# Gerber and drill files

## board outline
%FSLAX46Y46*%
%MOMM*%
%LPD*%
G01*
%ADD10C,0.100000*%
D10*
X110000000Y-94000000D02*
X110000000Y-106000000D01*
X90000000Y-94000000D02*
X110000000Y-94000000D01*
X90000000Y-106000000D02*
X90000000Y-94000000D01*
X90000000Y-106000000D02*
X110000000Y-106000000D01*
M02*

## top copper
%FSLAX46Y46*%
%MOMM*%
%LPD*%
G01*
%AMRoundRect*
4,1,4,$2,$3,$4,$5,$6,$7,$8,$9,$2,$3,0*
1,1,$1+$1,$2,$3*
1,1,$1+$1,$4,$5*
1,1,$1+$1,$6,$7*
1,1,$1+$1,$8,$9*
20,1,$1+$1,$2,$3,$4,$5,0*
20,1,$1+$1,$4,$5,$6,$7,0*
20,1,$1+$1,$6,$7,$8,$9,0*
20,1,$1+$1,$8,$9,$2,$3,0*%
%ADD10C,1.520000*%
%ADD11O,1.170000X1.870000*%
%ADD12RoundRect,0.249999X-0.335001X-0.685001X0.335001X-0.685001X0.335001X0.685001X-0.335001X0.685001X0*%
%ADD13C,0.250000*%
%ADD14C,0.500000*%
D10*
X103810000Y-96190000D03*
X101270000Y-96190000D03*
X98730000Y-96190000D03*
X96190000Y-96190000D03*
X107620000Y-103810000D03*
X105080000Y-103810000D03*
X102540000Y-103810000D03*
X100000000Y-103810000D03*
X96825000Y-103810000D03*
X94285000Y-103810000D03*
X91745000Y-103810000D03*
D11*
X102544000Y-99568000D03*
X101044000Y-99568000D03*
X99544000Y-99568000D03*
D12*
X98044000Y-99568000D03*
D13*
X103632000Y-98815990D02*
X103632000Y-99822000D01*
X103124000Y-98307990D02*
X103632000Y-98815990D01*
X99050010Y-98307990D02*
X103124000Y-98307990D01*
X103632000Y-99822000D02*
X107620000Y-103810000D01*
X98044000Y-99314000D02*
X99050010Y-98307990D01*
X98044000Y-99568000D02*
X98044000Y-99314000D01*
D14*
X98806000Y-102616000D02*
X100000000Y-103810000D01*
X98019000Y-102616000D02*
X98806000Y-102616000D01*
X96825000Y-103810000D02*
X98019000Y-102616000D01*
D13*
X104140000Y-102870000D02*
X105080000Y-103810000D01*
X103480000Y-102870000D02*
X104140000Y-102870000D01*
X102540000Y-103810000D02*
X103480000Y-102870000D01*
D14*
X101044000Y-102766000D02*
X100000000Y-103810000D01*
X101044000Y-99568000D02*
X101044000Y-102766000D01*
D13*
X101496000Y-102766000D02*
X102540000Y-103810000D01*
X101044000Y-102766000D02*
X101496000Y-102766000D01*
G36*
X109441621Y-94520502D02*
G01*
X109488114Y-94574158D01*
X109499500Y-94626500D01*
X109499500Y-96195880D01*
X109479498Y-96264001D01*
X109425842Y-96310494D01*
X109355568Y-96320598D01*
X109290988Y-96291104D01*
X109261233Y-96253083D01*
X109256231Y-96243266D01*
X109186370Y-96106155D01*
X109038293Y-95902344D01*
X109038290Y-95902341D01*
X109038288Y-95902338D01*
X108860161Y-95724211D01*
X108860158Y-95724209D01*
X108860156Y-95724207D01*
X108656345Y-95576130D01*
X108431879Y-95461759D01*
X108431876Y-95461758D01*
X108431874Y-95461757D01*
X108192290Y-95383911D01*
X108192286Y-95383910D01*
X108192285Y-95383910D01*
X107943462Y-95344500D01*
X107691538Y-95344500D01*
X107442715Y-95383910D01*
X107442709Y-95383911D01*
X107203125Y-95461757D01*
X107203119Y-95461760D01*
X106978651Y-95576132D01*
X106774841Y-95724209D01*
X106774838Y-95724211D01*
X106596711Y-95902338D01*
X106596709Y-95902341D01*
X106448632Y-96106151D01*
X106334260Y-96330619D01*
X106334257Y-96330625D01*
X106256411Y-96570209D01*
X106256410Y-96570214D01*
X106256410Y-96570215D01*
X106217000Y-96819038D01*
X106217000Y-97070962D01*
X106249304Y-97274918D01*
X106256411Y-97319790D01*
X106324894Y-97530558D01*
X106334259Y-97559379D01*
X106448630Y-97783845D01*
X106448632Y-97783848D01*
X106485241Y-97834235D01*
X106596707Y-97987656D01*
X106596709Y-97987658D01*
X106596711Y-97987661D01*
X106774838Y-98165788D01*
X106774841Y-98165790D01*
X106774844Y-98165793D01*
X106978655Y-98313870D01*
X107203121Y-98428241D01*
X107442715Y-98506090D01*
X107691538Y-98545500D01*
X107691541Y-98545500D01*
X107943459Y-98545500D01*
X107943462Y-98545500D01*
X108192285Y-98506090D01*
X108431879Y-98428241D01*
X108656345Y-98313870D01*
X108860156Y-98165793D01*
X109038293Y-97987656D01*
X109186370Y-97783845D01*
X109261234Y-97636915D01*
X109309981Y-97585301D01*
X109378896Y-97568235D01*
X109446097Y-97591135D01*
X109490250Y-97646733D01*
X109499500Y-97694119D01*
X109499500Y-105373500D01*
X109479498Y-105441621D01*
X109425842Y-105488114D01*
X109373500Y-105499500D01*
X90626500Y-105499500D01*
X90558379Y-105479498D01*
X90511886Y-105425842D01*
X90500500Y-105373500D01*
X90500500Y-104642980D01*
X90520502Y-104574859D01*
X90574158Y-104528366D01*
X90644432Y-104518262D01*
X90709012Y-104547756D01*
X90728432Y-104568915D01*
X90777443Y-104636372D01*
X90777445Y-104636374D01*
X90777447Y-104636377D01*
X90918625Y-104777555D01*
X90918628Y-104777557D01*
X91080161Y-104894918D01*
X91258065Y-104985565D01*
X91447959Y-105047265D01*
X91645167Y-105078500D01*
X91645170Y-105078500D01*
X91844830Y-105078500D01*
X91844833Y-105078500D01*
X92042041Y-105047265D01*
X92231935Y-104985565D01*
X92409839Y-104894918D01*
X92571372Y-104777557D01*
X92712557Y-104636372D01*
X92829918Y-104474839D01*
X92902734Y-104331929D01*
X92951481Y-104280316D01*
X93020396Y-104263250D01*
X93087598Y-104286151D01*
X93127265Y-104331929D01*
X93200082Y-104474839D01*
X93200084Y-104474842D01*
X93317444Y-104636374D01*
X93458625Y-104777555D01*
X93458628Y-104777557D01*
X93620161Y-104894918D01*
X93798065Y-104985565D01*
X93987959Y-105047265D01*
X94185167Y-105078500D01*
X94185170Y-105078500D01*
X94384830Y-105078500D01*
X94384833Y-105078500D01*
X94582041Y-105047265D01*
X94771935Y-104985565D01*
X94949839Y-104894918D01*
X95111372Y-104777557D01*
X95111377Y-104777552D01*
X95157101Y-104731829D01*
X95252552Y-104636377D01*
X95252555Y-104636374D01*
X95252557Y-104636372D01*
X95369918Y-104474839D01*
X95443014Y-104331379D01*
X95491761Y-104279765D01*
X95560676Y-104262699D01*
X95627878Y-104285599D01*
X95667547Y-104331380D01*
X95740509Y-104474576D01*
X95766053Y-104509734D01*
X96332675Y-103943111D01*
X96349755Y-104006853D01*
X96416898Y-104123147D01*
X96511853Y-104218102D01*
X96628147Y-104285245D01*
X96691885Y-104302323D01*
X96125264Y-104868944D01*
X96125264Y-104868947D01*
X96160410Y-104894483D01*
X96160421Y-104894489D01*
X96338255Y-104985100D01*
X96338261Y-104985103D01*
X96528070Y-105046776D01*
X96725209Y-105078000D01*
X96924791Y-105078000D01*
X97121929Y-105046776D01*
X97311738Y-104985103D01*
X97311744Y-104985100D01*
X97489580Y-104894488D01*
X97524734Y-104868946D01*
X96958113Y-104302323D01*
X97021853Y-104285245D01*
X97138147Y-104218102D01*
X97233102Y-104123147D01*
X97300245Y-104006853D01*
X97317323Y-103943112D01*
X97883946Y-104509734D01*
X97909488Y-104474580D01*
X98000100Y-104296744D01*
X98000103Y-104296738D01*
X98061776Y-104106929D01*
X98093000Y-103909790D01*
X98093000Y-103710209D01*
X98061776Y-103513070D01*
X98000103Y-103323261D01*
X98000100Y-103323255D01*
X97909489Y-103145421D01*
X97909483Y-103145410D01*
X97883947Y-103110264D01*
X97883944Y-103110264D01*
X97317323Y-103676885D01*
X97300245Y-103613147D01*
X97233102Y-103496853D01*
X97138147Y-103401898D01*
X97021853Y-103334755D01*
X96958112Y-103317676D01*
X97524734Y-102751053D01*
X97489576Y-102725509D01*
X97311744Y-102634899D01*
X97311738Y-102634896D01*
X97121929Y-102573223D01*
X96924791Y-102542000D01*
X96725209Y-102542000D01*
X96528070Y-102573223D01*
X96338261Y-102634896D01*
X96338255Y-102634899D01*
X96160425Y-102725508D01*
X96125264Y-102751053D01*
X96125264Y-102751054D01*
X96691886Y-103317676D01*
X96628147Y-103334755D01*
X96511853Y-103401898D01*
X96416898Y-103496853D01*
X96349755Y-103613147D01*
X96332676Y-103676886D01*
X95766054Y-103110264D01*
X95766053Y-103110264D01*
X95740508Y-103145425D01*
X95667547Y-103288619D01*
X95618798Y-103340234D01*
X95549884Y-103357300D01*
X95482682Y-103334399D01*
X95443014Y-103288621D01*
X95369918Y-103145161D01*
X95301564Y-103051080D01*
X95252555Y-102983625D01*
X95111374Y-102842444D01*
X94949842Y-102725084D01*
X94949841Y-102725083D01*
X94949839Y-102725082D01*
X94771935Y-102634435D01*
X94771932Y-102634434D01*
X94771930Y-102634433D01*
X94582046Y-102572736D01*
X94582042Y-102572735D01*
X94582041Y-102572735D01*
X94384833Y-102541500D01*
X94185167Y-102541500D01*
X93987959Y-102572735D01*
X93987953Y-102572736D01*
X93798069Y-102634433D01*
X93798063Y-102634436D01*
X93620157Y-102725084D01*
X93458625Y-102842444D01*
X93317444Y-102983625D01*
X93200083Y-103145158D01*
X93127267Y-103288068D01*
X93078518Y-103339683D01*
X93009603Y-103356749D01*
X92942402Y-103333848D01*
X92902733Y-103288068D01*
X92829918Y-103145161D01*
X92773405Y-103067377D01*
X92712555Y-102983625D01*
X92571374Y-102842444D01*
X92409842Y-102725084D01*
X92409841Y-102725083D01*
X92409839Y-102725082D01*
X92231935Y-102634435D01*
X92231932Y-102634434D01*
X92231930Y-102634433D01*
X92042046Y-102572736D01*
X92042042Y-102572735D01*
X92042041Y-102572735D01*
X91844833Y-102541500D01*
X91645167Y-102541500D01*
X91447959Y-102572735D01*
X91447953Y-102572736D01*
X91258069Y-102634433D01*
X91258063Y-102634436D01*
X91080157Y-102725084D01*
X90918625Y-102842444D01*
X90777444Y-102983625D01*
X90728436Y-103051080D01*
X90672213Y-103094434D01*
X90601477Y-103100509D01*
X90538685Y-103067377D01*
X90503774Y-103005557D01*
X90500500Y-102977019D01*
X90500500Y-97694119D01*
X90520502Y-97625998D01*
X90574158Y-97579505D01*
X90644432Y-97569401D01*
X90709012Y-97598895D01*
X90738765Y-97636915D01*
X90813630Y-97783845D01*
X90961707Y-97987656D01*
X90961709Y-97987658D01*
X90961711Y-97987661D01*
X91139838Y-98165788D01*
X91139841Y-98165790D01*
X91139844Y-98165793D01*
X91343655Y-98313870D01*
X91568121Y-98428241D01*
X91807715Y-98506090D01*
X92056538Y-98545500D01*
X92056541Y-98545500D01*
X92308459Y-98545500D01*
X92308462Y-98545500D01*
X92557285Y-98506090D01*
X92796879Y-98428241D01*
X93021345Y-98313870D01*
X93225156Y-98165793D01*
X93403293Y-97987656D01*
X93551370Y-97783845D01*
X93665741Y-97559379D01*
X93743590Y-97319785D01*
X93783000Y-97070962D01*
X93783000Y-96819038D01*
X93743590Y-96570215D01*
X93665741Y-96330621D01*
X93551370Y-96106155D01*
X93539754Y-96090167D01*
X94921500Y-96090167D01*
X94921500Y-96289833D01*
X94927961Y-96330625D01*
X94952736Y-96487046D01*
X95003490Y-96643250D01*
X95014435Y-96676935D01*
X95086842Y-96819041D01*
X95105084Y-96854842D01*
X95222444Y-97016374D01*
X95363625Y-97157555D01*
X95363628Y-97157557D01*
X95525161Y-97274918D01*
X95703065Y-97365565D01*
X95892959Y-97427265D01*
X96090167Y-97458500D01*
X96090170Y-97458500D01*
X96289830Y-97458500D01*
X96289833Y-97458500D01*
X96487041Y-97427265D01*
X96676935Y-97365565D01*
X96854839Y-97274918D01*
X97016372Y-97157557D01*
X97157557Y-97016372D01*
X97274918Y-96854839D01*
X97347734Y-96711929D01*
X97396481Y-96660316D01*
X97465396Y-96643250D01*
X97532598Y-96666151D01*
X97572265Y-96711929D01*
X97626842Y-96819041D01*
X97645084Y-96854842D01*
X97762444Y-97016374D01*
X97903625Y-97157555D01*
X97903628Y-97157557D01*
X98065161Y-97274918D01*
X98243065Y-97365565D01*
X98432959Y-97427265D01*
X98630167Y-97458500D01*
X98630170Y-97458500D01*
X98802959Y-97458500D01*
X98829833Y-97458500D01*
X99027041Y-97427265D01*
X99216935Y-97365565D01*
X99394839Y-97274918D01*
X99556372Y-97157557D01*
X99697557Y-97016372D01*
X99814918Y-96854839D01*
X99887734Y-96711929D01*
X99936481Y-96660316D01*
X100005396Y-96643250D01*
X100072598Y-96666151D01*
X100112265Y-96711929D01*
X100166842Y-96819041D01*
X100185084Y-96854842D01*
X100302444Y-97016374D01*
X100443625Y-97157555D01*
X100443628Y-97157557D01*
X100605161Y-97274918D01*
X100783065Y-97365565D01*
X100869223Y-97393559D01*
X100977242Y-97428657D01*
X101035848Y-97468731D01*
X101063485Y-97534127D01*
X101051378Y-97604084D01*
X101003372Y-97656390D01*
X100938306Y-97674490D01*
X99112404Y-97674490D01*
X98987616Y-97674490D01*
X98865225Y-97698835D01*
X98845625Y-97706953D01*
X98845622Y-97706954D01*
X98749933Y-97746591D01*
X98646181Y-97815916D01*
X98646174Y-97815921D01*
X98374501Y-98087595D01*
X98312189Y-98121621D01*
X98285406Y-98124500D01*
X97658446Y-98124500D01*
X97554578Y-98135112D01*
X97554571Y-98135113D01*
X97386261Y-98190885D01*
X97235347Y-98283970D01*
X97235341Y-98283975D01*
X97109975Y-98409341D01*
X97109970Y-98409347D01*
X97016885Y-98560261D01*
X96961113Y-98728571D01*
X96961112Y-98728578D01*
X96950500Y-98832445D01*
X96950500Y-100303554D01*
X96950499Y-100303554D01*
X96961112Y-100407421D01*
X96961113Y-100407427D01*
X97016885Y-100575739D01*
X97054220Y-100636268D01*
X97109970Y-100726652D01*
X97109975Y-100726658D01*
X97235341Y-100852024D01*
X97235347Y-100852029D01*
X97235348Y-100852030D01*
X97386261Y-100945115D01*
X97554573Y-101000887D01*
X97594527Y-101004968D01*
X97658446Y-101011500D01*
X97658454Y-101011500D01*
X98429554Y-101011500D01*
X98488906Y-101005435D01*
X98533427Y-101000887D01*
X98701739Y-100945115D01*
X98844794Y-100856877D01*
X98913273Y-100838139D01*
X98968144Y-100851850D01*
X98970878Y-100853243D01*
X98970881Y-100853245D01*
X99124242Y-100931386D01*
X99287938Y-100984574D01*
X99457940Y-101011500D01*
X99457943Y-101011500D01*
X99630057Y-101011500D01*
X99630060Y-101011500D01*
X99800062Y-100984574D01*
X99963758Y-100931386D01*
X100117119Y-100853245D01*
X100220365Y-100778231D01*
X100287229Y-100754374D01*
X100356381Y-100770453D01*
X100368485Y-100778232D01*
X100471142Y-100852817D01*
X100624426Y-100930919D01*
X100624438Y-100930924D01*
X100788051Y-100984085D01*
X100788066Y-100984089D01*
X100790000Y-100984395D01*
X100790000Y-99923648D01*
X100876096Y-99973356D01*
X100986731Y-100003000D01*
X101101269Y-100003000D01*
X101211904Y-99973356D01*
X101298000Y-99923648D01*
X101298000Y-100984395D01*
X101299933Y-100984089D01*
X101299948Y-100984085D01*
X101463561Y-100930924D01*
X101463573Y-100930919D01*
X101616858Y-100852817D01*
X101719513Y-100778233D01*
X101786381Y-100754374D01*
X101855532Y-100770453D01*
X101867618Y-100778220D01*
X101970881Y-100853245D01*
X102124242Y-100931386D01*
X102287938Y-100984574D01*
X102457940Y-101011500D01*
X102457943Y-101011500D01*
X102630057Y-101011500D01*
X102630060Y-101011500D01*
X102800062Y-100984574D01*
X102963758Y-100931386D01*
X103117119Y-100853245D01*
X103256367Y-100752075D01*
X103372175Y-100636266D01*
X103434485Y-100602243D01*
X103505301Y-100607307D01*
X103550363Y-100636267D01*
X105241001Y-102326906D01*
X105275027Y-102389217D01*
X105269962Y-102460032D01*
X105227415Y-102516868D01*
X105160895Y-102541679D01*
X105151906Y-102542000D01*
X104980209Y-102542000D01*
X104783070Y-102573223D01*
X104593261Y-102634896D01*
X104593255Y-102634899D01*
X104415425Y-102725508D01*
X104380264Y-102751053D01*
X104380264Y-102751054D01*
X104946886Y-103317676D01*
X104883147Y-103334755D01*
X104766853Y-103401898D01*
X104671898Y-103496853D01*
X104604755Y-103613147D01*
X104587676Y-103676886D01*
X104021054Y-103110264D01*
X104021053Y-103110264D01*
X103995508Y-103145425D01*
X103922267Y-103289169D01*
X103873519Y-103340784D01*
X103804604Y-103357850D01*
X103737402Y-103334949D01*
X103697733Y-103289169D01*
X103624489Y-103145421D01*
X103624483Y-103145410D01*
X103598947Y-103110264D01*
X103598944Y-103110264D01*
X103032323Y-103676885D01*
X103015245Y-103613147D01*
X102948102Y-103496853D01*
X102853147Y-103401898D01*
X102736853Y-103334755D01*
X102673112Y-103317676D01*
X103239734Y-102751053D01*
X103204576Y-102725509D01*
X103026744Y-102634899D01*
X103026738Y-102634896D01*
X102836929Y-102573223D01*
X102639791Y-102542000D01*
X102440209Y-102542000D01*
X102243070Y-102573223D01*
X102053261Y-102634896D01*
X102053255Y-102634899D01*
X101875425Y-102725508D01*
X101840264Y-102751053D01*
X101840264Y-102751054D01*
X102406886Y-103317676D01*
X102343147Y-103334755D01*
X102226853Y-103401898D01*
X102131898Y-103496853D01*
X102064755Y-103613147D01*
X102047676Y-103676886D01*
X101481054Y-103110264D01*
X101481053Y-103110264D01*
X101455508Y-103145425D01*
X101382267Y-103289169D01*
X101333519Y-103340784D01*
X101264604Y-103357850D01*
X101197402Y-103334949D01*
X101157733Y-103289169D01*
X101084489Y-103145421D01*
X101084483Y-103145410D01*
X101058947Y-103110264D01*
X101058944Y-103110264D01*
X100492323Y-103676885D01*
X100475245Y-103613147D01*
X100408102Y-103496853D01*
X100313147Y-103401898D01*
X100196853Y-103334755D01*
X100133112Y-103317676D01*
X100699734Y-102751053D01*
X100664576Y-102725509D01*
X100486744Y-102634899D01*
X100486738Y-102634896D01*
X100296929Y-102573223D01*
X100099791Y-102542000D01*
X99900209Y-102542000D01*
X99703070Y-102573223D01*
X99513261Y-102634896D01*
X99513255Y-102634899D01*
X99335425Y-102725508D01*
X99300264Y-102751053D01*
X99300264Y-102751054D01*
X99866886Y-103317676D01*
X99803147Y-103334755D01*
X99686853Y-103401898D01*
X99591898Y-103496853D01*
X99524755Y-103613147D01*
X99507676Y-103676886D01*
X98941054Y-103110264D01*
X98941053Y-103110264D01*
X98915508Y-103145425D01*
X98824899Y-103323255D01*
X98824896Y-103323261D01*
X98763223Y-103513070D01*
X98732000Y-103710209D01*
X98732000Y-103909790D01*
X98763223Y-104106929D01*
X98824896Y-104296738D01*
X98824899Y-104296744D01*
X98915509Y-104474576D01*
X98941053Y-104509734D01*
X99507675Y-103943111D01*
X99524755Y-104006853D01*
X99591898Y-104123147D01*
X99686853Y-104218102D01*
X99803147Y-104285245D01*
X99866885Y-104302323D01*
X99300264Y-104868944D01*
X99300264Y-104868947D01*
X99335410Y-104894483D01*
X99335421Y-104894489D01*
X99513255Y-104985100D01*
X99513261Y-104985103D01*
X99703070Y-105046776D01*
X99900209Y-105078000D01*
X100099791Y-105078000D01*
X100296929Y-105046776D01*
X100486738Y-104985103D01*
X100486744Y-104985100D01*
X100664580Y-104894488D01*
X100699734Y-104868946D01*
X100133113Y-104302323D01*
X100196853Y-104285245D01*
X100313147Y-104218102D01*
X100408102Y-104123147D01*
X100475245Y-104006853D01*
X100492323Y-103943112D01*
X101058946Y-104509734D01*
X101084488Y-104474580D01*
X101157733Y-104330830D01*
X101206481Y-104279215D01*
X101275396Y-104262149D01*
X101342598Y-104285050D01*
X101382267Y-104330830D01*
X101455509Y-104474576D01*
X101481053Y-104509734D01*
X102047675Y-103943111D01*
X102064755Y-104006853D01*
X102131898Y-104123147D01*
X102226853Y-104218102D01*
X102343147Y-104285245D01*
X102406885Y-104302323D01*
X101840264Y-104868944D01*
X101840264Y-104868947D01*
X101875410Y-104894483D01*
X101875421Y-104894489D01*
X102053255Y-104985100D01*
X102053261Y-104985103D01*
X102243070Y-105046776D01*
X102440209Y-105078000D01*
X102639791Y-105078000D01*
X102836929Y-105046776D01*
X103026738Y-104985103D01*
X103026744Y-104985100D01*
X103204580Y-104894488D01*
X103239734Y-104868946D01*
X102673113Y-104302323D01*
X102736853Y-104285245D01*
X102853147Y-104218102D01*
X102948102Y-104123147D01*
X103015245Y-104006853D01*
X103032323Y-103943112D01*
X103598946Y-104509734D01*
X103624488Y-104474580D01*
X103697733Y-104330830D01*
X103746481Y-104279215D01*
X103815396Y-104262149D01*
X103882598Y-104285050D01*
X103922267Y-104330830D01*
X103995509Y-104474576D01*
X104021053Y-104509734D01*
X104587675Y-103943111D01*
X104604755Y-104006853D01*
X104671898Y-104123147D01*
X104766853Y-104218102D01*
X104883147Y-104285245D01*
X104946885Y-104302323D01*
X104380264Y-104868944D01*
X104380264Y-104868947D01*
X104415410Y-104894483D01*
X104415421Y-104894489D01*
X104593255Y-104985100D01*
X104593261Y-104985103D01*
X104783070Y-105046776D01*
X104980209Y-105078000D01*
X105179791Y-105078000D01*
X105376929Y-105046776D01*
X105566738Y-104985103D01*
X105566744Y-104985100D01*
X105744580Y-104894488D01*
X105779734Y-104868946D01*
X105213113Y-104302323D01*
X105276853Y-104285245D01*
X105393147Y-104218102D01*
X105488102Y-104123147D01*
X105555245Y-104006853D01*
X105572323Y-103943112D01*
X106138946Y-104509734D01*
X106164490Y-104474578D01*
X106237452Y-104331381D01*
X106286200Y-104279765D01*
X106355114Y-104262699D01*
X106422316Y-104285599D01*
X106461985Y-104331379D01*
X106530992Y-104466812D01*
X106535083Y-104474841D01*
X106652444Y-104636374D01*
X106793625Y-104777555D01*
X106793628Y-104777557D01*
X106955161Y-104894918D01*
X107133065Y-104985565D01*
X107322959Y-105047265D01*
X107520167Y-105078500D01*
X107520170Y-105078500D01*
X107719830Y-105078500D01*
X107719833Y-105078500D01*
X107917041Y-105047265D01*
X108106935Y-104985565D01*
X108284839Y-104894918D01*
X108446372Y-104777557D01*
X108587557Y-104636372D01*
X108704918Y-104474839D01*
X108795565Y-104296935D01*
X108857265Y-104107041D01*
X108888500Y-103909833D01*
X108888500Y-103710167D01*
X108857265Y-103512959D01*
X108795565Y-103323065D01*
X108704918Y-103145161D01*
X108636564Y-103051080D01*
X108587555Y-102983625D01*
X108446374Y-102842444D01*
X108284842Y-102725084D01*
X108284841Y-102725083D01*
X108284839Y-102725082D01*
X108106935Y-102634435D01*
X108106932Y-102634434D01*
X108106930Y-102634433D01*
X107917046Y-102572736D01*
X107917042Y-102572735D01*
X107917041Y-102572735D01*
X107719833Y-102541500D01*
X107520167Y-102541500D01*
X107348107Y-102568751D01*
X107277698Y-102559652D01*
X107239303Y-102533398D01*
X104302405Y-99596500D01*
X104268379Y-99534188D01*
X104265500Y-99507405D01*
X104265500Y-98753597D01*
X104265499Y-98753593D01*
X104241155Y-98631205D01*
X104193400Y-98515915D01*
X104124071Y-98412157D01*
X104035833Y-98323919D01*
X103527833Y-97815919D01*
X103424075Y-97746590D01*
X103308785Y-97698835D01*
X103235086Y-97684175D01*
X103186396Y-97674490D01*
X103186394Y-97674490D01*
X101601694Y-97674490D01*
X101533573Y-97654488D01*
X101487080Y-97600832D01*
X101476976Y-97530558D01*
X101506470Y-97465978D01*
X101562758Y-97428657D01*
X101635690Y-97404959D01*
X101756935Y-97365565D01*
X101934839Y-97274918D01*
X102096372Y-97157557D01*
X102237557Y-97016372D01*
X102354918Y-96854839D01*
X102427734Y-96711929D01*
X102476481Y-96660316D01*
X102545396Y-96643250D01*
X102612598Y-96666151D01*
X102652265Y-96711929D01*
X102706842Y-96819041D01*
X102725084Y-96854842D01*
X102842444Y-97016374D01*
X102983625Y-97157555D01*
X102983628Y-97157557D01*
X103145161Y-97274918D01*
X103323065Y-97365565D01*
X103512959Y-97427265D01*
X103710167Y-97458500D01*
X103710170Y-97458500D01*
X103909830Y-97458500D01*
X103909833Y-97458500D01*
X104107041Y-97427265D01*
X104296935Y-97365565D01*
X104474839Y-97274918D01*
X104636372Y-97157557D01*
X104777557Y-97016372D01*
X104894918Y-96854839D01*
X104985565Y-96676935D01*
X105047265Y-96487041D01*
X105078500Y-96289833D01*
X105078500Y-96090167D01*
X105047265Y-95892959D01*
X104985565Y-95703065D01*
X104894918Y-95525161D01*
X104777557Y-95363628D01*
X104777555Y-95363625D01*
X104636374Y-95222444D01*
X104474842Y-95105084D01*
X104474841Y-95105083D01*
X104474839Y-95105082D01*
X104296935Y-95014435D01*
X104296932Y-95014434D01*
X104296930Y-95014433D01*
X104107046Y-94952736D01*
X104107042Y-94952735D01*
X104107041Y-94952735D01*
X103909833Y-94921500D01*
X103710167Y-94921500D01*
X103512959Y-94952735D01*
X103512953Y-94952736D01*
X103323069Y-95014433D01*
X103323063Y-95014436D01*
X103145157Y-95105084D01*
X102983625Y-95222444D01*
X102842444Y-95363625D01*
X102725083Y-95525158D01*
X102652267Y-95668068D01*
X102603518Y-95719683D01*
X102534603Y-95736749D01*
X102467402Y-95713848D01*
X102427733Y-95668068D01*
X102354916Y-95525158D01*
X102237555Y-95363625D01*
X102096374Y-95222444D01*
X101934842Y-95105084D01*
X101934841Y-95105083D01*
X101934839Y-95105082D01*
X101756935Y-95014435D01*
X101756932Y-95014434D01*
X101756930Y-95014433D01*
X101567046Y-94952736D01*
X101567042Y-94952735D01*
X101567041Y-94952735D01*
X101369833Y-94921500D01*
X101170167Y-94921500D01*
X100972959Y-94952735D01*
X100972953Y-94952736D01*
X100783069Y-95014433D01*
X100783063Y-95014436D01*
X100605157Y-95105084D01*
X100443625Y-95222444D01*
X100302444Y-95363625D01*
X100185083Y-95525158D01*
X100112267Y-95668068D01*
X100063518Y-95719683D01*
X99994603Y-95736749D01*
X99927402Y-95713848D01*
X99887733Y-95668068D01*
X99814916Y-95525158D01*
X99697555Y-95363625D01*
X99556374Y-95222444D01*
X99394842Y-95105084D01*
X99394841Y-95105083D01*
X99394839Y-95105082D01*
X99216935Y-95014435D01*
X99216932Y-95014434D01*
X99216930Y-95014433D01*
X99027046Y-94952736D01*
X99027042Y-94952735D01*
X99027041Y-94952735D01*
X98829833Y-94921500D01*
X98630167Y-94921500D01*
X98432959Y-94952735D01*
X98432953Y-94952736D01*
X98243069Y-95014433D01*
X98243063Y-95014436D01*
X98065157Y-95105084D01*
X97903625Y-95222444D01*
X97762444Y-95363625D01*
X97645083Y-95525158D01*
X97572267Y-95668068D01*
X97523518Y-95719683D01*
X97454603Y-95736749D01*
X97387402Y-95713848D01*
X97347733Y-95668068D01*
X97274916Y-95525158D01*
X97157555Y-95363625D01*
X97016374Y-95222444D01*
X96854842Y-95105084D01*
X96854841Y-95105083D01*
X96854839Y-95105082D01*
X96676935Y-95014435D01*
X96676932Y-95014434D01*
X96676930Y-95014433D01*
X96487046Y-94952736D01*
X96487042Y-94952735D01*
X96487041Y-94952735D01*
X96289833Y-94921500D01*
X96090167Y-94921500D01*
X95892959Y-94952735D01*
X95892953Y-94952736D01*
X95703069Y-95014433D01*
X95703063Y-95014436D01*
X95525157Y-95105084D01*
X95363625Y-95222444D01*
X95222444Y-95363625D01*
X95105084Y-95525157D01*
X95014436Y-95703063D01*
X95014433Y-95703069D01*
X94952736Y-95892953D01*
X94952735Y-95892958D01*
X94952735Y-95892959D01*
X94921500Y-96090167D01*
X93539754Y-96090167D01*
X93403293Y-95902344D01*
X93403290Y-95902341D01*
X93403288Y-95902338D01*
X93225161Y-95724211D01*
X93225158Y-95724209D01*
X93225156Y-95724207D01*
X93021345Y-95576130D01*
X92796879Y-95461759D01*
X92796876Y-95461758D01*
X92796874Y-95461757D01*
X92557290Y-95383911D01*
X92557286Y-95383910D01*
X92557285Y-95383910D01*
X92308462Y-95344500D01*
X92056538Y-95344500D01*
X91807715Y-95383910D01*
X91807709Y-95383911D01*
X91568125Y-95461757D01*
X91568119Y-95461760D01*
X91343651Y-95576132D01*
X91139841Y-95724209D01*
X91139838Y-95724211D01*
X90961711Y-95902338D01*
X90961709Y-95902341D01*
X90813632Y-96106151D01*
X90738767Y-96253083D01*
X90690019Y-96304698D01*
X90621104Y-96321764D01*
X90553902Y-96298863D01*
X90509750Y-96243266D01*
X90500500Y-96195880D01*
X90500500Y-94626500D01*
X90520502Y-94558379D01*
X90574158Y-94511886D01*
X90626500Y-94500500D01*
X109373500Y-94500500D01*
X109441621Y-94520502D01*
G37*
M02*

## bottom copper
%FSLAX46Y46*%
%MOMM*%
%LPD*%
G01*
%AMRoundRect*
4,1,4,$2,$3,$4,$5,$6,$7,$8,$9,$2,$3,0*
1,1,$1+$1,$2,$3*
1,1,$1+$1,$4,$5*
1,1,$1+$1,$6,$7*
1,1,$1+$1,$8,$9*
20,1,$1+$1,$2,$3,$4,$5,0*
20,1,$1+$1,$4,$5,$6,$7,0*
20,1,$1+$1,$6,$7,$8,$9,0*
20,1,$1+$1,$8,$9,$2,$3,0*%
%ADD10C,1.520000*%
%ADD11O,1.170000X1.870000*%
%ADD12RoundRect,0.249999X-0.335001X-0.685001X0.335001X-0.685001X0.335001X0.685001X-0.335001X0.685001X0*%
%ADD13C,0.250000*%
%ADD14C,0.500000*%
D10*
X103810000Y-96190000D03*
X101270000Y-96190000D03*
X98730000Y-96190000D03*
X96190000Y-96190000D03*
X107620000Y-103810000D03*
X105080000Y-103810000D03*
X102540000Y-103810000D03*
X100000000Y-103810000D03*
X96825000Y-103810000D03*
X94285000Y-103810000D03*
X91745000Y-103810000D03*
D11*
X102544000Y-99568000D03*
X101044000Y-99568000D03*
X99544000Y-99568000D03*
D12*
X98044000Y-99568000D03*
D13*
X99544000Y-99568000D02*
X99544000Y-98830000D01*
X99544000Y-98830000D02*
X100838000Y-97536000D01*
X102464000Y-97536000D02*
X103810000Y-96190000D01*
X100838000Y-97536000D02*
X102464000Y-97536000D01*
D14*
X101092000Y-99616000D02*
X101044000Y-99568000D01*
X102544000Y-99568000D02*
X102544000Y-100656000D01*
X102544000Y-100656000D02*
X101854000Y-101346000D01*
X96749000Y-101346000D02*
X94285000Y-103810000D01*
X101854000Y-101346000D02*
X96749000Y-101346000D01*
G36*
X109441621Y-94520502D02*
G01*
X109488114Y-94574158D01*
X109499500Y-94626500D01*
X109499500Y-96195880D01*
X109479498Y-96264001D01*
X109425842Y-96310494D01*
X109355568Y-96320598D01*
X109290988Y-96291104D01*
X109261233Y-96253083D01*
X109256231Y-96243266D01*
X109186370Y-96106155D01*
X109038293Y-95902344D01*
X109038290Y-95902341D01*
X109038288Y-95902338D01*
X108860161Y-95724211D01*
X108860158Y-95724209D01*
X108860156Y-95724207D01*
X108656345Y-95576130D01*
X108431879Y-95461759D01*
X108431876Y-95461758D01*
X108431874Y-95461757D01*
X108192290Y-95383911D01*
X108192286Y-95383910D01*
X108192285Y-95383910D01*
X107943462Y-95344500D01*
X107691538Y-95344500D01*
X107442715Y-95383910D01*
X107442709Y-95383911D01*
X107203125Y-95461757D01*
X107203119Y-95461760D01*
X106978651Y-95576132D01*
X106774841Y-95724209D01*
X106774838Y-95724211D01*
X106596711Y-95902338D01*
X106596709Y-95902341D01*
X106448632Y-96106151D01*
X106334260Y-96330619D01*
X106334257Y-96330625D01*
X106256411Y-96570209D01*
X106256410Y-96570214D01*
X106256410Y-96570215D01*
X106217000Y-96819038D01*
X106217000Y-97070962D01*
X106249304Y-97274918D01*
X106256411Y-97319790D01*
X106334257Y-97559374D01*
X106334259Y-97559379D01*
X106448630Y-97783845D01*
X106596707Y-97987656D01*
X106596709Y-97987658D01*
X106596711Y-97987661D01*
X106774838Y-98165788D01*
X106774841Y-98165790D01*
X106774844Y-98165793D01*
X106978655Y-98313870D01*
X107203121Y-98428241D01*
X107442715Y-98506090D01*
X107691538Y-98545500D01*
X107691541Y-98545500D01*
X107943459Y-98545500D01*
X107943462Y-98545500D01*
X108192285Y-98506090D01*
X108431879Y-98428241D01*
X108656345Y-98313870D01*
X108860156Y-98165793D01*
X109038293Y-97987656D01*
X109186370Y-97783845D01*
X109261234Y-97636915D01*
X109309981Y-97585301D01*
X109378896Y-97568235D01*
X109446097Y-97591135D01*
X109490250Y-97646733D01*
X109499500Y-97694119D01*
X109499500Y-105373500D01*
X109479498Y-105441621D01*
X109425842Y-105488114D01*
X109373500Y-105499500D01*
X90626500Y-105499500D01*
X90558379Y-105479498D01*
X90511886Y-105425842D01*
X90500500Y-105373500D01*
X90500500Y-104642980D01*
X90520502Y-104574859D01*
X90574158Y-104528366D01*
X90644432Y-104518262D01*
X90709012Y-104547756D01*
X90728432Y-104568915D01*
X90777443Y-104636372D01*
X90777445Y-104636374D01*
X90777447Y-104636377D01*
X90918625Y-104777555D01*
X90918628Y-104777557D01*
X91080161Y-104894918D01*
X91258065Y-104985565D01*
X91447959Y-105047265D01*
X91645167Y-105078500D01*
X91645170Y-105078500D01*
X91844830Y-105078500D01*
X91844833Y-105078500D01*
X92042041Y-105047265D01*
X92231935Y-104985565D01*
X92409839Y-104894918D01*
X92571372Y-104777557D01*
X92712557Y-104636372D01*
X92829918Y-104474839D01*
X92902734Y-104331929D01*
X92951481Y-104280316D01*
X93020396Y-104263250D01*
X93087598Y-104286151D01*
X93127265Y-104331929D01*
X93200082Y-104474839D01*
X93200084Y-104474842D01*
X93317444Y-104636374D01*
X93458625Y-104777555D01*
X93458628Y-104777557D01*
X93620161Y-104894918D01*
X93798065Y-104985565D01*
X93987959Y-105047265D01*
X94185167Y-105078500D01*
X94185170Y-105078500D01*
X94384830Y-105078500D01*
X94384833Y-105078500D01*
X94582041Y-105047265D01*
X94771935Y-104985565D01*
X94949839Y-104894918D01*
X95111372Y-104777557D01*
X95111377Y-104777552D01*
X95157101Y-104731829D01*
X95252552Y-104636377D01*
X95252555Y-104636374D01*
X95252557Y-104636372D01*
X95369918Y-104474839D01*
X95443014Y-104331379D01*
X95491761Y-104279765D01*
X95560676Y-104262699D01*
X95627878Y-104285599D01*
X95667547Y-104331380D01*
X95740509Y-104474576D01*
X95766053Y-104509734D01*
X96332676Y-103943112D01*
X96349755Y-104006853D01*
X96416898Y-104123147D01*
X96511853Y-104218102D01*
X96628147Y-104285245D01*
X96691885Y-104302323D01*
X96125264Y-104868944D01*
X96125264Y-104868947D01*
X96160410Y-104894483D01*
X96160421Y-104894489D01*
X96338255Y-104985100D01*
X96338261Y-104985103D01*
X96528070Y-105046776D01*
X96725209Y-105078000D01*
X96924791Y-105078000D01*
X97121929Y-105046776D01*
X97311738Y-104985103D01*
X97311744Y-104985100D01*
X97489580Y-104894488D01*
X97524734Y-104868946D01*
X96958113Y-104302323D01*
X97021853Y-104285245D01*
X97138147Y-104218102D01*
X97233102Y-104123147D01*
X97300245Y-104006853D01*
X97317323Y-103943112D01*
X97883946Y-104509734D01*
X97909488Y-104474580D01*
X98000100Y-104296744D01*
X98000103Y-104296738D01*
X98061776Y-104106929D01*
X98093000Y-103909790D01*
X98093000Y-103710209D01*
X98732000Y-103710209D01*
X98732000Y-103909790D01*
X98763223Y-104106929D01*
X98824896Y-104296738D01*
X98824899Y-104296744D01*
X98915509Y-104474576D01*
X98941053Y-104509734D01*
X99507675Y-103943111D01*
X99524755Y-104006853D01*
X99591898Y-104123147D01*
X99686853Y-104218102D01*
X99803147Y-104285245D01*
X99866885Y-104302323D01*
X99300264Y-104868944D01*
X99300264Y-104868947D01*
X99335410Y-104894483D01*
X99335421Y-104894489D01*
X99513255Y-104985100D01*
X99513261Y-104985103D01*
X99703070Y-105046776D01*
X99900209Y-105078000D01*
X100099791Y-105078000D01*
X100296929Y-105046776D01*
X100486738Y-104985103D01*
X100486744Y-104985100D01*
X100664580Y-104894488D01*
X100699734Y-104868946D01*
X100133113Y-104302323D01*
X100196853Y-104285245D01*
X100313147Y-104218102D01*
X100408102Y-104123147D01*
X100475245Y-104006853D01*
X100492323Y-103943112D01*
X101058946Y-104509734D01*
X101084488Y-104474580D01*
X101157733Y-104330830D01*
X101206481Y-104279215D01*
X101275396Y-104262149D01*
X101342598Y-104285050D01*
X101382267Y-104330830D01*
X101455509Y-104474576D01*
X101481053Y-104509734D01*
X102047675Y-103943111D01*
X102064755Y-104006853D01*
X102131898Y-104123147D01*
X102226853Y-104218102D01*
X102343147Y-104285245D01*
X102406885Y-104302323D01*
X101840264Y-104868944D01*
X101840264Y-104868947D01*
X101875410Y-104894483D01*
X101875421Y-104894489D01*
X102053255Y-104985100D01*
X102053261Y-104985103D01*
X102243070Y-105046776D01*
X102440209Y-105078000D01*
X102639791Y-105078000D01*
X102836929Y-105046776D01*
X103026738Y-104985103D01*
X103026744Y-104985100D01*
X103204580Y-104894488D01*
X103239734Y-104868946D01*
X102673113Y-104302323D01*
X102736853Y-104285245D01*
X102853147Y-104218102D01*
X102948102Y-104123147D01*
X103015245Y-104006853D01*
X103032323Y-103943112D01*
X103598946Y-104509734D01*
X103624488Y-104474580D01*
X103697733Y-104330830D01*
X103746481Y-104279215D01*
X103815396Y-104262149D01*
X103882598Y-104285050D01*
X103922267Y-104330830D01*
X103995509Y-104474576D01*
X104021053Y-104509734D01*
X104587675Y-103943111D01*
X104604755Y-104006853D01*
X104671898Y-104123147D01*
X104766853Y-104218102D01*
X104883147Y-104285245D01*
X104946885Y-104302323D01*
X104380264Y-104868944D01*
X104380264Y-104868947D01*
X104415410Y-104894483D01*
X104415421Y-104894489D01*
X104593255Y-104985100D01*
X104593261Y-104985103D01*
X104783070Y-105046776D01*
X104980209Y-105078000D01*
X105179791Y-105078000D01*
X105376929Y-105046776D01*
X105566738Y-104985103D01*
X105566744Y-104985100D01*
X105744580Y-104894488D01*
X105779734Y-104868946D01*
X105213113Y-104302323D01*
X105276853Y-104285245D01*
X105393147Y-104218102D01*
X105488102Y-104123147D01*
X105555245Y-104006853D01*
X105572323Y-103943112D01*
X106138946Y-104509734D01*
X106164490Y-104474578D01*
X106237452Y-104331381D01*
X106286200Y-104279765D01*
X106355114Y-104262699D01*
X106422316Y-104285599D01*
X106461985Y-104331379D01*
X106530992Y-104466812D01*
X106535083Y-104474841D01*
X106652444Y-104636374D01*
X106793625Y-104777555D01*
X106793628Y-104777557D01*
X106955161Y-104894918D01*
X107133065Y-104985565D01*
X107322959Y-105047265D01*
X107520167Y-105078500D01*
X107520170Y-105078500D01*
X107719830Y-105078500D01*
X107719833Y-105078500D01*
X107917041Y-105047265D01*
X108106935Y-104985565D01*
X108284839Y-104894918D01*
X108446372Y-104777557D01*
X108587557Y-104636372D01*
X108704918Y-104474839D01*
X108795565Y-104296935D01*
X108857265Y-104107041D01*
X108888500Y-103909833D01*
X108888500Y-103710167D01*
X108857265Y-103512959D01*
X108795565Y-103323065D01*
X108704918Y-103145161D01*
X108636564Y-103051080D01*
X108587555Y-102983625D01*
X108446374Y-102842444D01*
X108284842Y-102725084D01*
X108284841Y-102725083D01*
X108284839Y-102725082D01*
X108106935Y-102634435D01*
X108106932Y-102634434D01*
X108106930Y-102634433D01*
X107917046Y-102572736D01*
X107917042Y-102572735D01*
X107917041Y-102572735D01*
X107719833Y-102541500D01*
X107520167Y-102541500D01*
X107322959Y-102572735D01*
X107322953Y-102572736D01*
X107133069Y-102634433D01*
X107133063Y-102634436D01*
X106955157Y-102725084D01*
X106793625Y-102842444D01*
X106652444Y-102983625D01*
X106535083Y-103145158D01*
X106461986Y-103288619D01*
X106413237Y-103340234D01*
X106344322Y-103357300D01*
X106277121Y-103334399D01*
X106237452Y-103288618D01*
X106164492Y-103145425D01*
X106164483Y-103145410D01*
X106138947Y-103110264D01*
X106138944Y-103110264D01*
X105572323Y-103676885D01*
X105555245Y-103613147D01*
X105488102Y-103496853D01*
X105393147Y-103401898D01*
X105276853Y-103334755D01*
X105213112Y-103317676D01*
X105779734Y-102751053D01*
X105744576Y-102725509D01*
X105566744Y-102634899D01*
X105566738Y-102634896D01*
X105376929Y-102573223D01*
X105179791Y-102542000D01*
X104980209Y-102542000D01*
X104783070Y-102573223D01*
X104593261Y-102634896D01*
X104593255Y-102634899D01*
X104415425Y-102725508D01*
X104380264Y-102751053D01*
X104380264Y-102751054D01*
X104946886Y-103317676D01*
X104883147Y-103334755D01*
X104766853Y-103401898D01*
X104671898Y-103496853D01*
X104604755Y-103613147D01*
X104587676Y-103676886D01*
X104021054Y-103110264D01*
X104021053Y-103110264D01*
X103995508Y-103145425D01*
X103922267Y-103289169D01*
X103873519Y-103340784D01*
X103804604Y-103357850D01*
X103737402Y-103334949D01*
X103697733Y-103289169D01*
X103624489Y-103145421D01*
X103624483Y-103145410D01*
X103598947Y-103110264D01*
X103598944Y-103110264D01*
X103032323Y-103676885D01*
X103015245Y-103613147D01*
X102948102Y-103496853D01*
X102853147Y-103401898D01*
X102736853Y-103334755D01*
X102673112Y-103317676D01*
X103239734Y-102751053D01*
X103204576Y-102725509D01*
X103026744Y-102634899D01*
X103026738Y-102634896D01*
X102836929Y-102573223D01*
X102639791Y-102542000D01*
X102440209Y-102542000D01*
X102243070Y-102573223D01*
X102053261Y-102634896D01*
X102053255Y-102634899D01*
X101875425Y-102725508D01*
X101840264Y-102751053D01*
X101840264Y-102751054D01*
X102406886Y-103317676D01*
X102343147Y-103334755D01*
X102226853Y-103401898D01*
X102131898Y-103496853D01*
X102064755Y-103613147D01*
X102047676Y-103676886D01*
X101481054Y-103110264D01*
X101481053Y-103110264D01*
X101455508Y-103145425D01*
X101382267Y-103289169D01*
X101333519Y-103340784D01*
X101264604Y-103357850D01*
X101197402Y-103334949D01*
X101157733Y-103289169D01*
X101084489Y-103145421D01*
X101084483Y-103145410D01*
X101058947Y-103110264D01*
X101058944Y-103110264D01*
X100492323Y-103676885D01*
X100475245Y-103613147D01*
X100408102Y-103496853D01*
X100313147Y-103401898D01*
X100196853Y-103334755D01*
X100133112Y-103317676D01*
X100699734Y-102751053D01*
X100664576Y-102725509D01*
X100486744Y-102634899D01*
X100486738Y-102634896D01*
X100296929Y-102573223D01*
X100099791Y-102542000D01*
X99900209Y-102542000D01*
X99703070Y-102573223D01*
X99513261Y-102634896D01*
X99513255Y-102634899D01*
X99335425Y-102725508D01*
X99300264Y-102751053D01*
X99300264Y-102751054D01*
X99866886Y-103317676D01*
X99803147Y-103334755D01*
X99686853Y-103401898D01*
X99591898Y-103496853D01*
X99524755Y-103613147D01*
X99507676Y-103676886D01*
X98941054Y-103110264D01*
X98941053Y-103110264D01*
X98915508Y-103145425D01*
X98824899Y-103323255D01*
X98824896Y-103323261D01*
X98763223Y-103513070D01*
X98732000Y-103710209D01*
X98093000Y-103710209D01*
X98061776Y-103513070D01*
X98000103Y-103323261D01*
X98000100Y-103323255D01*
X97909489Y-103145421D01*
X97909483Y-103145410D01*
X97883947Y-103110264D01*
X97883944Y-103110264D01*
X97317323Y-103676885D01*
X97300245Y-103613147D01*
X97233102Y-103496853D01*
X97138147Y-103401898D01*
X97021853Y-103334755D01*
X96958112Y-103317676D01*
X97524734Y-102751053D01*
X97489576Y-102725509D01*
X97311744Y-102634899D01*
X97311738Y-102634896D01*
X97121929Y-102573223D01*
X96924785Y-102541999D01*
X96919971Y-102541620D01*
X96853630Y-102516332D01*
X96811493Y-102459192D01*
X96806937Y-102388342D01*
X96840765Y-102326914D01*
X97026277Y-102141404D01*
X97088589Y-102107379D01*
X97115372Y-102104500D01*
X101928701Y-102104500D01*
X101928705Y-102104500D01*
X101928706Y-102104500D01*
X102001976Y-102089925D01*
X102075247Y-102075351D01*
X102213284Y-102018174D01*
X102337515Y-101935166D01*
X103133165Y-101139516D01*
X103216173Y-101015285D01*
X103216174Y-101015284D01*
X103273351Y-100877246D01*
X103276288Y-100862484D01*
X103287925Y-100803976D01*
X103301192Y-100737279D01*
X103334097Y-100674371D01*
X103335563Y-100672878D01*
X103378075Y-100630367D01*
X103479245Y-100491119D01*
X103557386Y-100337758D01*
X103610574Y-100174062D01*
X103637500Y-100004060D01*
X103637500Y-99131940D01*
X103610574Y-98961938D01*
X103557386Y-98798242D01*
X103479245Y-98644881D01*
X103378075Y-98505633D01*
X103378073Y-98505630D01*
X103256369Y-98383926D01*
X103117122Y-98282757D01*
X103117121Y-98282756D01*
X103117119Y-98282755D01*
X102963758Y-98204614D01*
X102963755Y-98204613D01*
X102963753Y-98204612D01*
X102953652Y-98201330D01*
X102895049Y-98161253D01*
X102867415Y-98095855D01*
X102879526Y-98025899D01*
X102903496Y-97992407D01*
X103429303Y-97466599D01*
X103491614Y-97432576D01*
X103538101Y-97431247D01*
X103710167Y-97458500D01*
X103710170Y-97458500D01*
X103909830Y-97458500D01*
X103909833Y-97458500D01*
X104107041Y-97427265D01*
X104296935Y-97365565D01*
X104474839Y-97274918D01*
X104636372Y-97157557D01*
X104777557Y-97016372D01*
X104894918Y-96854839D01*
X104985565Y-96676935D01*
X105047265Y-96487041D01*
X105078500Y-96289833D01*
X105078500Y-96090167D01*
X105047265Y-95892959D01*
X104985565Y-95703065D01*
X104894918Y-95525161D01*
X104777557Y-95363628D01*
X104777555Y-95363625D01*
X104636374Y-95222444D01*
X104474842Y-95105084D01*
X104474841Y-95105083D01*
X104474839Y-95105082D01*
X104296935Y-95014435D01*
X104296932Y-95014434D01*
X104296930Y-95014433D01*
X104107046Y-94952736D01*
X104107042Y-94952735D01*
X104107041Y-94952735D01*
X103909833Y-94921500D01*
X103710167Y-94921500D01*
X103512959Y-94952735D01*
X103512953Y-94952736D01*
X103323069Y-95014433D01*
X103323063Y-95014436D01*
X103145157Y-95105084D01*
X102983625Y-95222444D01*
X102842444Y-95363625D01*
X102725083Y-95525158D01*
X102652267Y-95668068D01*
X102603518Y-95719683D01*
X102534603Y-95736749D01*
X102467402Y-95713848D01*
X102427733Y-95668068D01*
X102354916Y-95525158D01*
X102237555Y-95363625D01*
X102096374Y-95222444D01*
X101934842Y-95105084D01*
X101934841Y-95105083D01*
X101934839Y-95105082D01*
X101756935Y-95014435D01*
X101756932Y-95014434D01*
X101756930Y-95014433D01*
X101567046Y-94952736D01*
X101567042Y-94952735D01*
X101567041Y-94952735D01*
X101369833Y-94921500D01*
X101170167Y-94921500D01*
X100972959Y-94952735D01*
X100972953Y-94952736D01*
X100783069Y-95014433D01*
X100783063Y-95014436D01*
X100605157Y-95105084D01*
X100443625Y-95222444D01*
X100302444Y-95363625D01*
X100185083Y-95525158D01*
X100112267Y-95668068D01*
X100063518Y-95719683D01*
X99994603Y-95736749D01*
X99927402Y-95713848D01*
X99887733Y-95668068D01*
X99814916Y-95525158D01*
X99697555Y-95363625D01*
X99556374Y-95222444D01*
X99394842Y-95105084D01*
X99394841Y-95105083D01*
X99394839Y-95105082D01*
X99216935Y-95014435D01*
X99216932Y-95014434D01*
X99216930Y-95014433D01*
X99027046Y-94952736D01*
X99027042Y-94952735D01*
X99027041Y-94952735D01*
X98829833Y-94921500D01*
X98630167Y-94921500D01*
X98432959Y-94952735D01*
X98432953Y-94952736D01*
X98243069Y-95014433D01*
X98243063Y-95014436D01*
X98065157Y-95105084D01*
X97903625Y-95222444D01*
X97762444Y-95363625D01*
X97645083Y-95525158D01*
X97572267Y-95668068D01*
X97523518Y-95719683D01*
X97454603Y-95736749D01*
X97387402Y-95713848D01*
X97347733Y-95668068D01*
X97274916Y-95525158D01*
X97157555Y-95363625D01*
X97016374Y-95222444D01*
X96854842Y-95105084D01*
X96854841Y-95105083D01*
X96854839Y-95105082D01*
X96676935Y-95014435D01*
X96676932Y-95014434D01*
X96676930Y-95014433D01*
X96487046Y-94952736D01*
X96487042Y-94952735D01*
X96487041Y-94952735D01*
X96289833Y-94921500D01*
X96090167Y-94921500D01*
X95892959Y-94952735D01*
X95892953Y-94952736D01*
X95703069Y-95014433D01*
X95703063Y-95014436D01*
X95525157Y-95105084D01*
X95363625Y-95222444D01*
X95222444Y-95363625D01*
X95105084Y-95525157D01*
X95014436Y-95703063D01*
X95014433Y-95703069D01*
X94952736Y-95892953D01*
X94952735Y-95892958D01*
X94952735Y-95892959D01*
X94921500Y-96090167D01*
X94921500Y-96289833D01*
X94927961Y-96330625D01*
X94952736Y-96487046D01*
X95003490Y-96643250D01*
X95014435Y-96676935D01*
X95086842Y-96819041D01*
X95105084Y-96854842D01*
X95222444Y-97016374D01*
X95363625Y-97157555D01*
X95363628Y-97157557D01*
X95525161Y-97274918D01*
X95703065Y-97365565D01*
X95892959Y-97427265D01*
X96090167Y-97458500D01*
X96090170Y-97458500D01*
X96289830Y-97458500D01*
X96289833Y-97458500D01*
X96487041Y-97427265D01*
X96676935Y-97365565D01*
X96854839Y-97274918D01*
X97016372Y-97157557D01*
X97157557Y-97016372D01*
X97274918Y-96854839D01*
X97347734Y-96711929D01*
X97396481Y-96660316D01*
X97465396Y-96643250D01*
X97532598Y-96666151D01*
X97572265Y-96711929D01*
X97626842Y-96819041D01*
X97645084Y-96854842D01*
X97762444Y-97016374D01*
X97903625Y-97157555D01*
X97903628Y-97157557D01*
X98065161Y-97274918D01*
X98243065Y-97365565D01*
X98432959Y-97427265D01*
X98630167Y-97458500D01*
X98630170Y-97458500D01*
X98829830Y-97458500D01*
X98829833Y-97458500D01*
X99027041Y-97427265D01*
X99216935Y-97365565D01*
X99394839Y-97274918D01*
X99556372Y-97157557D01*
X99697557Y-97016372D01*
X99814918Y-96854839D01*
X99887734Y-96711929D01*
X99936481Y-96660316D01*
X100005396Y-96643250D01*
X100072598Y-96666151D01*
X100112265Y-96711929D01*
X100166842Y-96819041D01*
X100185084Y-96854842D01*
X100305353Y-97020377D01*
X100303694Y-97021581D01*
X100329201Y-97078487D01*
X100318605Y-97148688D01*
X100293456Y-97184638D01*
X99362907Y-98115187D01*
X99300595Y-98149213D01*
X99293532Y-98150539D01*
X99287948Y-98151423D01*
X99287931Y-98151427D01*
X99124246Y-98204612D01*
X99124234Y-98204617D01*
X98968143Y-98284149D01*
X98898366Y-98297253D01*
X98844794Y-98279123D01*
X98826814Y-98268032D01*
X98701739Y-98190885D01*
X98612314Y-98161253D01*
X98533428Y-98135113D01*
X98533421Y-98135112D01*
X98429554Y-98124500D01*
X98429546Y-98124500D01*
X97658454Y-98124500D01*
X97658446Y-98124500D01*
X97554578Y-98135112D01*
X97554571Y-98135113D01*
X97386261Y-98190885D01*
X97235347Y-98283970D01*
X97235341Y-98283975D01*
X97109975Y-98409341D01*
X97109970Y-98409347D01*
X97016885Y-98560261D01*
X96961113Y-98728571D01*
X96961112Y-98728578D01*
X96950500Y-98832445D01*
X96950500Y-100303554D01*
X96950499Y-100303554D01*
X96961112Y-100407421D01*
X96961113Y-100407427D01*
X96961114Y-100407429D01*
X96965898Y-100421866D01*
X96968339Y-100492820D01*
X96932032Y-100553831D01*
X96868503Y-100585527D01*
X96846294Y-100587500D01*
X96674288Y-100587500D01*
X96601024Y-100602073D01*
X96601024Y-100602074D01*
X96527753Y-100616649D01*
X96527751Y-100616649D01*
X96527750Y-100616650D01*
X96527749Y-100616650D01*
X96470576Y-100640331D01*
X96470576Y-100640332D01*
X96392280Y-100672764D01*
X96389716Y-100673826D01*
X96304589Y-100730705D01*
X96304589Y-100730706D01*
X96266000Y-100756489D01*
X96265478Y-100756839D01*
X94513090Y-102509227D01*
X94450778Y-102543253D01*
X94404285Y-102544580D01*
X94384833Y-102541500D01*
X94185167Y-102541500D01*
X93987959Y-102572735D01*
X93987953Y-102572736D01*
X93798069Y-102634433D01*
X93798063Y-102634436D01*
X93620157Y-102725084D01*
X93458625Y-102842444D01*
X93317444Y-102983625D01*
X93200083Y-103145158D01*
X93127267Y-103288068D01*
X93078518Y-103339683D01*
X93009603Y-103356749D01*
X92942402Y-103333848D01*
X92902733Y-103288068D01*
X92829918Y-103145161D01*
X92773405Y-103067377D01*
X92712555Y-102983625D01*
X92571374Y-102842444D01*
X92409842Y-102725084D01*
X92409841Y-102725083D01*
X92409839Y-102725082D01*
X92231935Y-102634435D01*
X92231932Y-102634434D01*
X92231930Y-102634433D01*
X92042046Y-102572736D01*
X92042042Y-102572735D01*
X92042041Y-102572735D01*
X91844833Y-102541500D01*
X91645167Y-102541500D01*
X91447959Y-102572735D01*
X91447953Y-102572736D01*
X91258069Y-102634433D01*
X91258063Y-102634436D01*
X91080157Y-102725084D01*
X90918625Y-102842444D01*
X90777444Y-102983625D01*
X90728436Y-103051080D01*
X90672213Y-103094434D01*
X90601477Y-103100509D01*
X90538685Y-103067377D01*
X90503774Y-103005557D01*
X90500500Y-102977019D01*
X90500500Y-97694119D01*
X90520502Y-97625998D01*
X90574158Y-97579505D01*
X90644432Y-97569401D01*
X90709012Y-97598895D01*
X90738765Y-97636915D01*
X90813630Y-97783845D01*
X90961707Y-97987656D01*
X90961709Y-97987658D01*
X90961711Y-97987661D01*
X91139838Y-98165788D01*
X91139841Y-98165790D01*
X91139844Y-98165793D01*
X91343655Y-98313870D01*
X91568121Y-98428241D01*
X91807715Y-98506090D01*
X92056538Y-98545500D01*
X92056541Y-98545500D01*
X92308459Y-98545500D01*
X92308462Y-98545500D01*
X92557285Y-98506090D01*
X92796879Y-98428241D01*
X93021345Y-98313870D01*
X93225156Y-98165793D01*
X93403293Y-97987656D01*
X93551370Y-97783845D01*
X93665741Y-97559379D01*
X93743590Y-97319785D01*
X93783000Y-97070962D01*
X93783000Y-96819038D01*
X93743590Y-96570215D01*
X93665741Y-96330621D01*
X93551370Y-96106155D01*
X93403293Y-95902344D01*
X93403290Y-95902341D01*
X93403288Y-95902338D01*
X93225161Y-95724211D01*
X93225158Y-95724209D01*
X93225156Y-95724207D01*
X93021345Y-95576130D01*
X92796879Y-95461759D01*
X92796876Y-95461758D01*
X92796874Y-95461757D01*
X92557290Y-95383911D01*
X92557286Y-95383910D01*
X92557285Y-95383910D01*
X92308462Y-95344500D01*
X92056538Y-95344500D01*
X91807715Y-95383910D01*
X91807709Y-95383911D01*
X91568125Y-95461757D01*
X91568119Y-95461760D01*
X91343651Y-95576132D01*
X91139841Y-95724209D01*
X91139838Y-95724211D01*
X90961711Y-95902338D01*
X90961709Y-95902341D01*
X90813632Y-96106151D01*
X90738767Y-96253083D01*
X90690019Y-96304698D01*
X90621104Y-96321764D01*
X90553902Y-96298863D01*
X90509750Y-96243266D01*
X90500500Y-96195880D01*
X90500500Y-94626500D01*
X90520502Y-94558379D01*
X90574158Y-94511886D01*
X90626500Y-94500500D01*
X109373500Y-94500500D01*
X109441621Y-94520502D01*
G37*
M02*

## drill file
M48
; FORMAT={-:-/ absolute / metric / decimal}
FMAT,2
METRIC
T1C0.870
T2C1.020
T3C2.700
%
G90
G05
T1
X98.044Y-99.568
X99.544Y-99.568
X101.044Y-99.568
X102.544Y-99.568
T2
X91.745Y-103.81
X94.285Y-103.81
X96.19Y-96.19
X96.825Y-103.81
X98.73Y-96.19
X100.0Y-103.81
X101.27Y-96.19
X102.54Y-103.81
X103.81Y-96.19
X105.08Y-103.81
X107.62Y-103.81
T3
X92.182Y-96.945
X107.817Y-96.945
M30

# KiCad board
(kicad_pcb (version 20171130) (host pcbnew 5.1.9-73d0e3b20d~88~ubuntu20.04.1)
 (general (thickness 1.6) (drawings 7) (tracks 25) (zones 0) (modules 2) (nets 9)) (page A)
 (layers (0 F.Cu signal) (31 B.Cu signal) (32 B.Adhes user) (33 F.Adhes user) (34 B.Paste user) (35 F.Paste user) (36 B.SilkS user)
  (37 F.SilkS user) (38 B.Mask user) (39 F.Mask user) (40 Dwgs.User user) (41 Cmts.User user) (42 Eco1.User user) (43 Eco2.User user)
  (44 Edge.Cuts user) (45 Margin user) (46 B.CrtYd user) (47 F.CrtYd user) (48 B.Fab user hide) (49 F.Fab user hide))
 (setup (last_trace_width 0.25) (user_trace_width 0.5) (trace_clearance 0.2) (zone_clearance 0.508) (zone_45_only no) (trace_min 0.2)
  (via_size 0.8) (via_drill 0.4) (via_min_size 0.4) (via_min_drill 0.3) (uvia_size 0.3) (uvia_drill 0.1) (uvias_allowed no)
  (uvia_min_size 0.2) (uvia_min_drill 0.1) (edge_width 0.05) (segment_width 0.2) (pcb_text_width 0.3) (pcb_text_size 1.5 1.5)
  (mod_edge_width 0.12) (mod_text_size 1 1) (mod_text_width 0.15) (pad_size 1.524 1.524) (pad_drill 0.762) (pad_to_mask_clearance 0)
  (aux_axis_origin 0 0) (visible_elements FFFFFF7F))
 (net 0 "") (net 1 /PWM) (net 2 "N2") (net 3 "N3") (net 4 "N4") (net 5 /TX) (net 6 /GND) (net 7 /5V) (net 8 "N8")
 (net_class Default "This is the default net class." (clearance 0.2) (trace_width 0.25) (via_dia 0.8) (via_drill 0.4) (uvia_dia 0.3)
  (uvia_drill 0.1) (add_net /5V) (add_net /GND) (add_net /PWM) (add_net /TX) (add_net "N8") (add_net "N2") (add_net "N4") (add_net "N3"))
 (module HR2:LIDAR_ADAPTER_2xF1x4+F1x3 (layer F.Cu) (at 100 100)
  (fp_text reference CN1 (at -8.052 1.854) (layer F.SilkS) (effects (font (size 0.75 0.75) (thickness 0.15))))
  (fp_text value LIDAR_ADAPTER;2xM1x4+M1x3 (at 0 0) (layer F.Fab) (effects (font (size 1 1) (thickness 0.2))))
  (pad "West Lidar Mount Hole" np_thru_hole circle (at -7.8175 -3.055) (size 2.7 2.7) (drill 2.7) (layers *.Cu *.Mask))
  (pad "East Lidar Mount Hole" np_thru_hole circle (at 7.8175 -3.055) (size 2.7 2.7) (drill 2.7) (layers *.Cu *.Mask))
  (pad 11 thru_hole circle (at 3.81 -3.81) (size 1.52 1.52) (drill 1.02) (layers *.Cu *.Mask) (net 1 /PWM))
  (pad 10 thru_hole circle (at 1.27 -3.81) (size 1.52 1.52) (drill 1.02) (layers *.Cu *.Mask) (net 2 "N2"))
  (pad 9 thru_hole circle (at -1.27 -3.81) (size 1.52 1.52) (drill 1.02) (layers *.Cu *.Mask) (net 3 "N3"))
  (pad 8 thru_hole circle (at -3.81 -3.81) (size 1.52 1.52) (drill 1.02) (layers *.Cu *.Mask) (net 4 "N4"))
  (pad 7 thru_hole circle (at 7.62 3.81) (size 1.52 1.52) (drill 1.02) (layers *.Cu *.Mask) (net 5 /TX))
  (pad 6 thru_hole circle (at 5.08 3.81) (size 1.52 1.52) (drill 1.02) (layers *.Cu *.Mask) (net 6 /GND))
  (pad 5 thru_hole circle (at 2.54 3.81) (size 1.52 1.52) (drill 1.02) (layers *.Cu *.Mask) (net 6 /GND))
  (pad 4 thru_hole circle (at 0 3.81) (size 1.52 1.52) (drill 1.02) (layers *.Cu *.Mask) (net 6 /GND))
  (pad 3 thru_hole circle (at -3.175 3.81) (size 1.52 1.52) (drill 1.02) (layers *.Cu *.Mask) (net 6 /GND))
  (pad 2 thru_hole circle (at -5.715 3.81) (size 1.52 1.52) (drill 1.02) (layers *.Cu *.Mask) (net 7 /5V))
  (pad 1 thru_hole circle (at -8.255 3.81) (size 1.52 1.52) (drill 1.02) (layers *.Cu *.Mask) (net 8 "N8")))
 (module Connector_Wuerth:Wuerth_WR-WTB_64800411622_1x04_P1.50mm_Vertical (layer F.Cu) (at 98.044 99.568)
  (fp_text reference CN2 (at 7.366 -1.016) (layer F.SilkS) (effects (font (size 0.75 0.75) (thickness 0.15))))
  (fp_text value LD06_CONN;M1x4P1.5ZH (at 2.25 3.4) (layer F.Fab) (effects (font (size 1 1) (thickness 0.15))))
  (pad 4 thru_hole oval (at 4.5 0) (size 1.17 1.87) (drill 0.87) (layers *.Cu *.Mask) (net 7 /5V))
  (pad 3 thru_hole oval (at 3 0) (size 1.17 1.87) (drill 0.87) (layers *.Cu *.Mask) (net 6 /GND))
  (pad 2 thru_hole oval (at 1.5 0) (size 1.17 1.87) (drill 0.87) (layers *.Cu *.Mask) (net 1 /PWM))
  (pad 1 thru_hole roundrect (at 0 0) (size 1.17 1.87) (drill 0.87) (layers *.Cu *.Mask) (roundrect_rratio 0.213674358974359) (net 5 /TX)))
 (gr_line (start 110 94) (end 110 106) (layer Edge.Cuts) (width 0.1))
 (gr_line (start 90 94) (end 110 94) (layer Edge.Cuts) (width 0.1))
 (gr_line (start 90 106) (end 90 94) (layer Edge.Cuts) (width 0.1))
 (gr_line (start 90 106) (end 110 106) (layer Edge.Cuts) (width 0.1))
 (segment (start 99.544 99.568) (end 99.544 98.83) (width 0.25) (layer B.Cu) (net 1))
 (segment (start 99.544 98.83) (end 100.838 97.536) (width 0.25) (layer B.Cu) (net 1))
 (segment (start 102.464 97.536) (end 103.81 96.19) (width 0.25) (layer B.Cu) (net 1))
 (segment (start 100.838 97.536) (end 102.464 97.536) (width 0.25) (layer B.Cu) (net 1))
 (segment (start 103.632 98.81599) (end 103.632 99.822) (width 0.25) (layer F.Cu) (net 5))
 (segment (start 103.124 98.30799) (end 103.632 98.81599) (width 0.25) (layer F.Cu) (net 5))
 (segment (start 99.05001 98.30799) (end 103.124 98.30799) (width 0.25) (layer F.Cu) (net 5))
 (segment (start 103.632 99.822) (end 107.62 103.81) (width 0.25) (layer F.Cu) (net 5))
 (segment (start 98.044 99.314) (end 99.05001 98.30799) (width 0.25) (layer F.Cu) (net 5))
 (segment (start 98.044 99.568) (end 98.044 99.314) (width 0.25) (layer F.Cu) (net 5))
 (segment (start 101.092 99.616) (end 101.044 99.568) (width 0.5) (layer B.Cu) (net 6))
 (segment (start 98.806 102.616) (end 100 103.81) (width 0.5) (layer F.Cu) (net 6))
 (segment (start 98.019 102.616) (end 98.806 102.616) (width 0.5) (layer F.Cu) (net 6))
 (segment (start 96.825 103.81) (end 98.019 102.616) (width 0.5) (layer F.Cu) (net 6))
 (segment (start 104.14 102.87) (end 105.08 103.81) (width 0.25) (layer F.Cu) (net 6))
 (segment (start 103.48 102.87) (end 104.14 102.87) (width 0.25) (layer F.Cu) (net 6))
 (segment (start 102.54 103.81) (end 103.48 102.87) (width 0.25) (layer F.Cu) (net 6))
 (segment (start 101.044 102.766) (end 100 103.81) (width 0.5) (layer F.Cu) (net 6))
 (segment (start 101.044 99.568) (end 101.044 102.766) (width 0.5) (layer F.Cu) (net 6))
 (segment (start 101.496 102.766) (end 102.54 103.81) (width 0.25) (layer F.Cu) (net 6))
 (segment (start 101.044 102.766) (end 101.496 102.766) (width 0.25) (layer F.Cu) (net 6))
 (segment (start 102.544 99.568) (end 102.544 100.656) (width 0.5) (layer B.Cu) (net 7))
 (segment (start 102.544 100.656) (end 101.854 101.346) (width 0.5) (layer B.Cu) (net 7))
 (segment (start 96.749 101.346) (end 94.285 103.81) (width 0.5) (layer B.Cu) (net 7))
 (segment (start 101.854 101.346) (end 96.749 101.346) (width 0.5) (layer B.Cu) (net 7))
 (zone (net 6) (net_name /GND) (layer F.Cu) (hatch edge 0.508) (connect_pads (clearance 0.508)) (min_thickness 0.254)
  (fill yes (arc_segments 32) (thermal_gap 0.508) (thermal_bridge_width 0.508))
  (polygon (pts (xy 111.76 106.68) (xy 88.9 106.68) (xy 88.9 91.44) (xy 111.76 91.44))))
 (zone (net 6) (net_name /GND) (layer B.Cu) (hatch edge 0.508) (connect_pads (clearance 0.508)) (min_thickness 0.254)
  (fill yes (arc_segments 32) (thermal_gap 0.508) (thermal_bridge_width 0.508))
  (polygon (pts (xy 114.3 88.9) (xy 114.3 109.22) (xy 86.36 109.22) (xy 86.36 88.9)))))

